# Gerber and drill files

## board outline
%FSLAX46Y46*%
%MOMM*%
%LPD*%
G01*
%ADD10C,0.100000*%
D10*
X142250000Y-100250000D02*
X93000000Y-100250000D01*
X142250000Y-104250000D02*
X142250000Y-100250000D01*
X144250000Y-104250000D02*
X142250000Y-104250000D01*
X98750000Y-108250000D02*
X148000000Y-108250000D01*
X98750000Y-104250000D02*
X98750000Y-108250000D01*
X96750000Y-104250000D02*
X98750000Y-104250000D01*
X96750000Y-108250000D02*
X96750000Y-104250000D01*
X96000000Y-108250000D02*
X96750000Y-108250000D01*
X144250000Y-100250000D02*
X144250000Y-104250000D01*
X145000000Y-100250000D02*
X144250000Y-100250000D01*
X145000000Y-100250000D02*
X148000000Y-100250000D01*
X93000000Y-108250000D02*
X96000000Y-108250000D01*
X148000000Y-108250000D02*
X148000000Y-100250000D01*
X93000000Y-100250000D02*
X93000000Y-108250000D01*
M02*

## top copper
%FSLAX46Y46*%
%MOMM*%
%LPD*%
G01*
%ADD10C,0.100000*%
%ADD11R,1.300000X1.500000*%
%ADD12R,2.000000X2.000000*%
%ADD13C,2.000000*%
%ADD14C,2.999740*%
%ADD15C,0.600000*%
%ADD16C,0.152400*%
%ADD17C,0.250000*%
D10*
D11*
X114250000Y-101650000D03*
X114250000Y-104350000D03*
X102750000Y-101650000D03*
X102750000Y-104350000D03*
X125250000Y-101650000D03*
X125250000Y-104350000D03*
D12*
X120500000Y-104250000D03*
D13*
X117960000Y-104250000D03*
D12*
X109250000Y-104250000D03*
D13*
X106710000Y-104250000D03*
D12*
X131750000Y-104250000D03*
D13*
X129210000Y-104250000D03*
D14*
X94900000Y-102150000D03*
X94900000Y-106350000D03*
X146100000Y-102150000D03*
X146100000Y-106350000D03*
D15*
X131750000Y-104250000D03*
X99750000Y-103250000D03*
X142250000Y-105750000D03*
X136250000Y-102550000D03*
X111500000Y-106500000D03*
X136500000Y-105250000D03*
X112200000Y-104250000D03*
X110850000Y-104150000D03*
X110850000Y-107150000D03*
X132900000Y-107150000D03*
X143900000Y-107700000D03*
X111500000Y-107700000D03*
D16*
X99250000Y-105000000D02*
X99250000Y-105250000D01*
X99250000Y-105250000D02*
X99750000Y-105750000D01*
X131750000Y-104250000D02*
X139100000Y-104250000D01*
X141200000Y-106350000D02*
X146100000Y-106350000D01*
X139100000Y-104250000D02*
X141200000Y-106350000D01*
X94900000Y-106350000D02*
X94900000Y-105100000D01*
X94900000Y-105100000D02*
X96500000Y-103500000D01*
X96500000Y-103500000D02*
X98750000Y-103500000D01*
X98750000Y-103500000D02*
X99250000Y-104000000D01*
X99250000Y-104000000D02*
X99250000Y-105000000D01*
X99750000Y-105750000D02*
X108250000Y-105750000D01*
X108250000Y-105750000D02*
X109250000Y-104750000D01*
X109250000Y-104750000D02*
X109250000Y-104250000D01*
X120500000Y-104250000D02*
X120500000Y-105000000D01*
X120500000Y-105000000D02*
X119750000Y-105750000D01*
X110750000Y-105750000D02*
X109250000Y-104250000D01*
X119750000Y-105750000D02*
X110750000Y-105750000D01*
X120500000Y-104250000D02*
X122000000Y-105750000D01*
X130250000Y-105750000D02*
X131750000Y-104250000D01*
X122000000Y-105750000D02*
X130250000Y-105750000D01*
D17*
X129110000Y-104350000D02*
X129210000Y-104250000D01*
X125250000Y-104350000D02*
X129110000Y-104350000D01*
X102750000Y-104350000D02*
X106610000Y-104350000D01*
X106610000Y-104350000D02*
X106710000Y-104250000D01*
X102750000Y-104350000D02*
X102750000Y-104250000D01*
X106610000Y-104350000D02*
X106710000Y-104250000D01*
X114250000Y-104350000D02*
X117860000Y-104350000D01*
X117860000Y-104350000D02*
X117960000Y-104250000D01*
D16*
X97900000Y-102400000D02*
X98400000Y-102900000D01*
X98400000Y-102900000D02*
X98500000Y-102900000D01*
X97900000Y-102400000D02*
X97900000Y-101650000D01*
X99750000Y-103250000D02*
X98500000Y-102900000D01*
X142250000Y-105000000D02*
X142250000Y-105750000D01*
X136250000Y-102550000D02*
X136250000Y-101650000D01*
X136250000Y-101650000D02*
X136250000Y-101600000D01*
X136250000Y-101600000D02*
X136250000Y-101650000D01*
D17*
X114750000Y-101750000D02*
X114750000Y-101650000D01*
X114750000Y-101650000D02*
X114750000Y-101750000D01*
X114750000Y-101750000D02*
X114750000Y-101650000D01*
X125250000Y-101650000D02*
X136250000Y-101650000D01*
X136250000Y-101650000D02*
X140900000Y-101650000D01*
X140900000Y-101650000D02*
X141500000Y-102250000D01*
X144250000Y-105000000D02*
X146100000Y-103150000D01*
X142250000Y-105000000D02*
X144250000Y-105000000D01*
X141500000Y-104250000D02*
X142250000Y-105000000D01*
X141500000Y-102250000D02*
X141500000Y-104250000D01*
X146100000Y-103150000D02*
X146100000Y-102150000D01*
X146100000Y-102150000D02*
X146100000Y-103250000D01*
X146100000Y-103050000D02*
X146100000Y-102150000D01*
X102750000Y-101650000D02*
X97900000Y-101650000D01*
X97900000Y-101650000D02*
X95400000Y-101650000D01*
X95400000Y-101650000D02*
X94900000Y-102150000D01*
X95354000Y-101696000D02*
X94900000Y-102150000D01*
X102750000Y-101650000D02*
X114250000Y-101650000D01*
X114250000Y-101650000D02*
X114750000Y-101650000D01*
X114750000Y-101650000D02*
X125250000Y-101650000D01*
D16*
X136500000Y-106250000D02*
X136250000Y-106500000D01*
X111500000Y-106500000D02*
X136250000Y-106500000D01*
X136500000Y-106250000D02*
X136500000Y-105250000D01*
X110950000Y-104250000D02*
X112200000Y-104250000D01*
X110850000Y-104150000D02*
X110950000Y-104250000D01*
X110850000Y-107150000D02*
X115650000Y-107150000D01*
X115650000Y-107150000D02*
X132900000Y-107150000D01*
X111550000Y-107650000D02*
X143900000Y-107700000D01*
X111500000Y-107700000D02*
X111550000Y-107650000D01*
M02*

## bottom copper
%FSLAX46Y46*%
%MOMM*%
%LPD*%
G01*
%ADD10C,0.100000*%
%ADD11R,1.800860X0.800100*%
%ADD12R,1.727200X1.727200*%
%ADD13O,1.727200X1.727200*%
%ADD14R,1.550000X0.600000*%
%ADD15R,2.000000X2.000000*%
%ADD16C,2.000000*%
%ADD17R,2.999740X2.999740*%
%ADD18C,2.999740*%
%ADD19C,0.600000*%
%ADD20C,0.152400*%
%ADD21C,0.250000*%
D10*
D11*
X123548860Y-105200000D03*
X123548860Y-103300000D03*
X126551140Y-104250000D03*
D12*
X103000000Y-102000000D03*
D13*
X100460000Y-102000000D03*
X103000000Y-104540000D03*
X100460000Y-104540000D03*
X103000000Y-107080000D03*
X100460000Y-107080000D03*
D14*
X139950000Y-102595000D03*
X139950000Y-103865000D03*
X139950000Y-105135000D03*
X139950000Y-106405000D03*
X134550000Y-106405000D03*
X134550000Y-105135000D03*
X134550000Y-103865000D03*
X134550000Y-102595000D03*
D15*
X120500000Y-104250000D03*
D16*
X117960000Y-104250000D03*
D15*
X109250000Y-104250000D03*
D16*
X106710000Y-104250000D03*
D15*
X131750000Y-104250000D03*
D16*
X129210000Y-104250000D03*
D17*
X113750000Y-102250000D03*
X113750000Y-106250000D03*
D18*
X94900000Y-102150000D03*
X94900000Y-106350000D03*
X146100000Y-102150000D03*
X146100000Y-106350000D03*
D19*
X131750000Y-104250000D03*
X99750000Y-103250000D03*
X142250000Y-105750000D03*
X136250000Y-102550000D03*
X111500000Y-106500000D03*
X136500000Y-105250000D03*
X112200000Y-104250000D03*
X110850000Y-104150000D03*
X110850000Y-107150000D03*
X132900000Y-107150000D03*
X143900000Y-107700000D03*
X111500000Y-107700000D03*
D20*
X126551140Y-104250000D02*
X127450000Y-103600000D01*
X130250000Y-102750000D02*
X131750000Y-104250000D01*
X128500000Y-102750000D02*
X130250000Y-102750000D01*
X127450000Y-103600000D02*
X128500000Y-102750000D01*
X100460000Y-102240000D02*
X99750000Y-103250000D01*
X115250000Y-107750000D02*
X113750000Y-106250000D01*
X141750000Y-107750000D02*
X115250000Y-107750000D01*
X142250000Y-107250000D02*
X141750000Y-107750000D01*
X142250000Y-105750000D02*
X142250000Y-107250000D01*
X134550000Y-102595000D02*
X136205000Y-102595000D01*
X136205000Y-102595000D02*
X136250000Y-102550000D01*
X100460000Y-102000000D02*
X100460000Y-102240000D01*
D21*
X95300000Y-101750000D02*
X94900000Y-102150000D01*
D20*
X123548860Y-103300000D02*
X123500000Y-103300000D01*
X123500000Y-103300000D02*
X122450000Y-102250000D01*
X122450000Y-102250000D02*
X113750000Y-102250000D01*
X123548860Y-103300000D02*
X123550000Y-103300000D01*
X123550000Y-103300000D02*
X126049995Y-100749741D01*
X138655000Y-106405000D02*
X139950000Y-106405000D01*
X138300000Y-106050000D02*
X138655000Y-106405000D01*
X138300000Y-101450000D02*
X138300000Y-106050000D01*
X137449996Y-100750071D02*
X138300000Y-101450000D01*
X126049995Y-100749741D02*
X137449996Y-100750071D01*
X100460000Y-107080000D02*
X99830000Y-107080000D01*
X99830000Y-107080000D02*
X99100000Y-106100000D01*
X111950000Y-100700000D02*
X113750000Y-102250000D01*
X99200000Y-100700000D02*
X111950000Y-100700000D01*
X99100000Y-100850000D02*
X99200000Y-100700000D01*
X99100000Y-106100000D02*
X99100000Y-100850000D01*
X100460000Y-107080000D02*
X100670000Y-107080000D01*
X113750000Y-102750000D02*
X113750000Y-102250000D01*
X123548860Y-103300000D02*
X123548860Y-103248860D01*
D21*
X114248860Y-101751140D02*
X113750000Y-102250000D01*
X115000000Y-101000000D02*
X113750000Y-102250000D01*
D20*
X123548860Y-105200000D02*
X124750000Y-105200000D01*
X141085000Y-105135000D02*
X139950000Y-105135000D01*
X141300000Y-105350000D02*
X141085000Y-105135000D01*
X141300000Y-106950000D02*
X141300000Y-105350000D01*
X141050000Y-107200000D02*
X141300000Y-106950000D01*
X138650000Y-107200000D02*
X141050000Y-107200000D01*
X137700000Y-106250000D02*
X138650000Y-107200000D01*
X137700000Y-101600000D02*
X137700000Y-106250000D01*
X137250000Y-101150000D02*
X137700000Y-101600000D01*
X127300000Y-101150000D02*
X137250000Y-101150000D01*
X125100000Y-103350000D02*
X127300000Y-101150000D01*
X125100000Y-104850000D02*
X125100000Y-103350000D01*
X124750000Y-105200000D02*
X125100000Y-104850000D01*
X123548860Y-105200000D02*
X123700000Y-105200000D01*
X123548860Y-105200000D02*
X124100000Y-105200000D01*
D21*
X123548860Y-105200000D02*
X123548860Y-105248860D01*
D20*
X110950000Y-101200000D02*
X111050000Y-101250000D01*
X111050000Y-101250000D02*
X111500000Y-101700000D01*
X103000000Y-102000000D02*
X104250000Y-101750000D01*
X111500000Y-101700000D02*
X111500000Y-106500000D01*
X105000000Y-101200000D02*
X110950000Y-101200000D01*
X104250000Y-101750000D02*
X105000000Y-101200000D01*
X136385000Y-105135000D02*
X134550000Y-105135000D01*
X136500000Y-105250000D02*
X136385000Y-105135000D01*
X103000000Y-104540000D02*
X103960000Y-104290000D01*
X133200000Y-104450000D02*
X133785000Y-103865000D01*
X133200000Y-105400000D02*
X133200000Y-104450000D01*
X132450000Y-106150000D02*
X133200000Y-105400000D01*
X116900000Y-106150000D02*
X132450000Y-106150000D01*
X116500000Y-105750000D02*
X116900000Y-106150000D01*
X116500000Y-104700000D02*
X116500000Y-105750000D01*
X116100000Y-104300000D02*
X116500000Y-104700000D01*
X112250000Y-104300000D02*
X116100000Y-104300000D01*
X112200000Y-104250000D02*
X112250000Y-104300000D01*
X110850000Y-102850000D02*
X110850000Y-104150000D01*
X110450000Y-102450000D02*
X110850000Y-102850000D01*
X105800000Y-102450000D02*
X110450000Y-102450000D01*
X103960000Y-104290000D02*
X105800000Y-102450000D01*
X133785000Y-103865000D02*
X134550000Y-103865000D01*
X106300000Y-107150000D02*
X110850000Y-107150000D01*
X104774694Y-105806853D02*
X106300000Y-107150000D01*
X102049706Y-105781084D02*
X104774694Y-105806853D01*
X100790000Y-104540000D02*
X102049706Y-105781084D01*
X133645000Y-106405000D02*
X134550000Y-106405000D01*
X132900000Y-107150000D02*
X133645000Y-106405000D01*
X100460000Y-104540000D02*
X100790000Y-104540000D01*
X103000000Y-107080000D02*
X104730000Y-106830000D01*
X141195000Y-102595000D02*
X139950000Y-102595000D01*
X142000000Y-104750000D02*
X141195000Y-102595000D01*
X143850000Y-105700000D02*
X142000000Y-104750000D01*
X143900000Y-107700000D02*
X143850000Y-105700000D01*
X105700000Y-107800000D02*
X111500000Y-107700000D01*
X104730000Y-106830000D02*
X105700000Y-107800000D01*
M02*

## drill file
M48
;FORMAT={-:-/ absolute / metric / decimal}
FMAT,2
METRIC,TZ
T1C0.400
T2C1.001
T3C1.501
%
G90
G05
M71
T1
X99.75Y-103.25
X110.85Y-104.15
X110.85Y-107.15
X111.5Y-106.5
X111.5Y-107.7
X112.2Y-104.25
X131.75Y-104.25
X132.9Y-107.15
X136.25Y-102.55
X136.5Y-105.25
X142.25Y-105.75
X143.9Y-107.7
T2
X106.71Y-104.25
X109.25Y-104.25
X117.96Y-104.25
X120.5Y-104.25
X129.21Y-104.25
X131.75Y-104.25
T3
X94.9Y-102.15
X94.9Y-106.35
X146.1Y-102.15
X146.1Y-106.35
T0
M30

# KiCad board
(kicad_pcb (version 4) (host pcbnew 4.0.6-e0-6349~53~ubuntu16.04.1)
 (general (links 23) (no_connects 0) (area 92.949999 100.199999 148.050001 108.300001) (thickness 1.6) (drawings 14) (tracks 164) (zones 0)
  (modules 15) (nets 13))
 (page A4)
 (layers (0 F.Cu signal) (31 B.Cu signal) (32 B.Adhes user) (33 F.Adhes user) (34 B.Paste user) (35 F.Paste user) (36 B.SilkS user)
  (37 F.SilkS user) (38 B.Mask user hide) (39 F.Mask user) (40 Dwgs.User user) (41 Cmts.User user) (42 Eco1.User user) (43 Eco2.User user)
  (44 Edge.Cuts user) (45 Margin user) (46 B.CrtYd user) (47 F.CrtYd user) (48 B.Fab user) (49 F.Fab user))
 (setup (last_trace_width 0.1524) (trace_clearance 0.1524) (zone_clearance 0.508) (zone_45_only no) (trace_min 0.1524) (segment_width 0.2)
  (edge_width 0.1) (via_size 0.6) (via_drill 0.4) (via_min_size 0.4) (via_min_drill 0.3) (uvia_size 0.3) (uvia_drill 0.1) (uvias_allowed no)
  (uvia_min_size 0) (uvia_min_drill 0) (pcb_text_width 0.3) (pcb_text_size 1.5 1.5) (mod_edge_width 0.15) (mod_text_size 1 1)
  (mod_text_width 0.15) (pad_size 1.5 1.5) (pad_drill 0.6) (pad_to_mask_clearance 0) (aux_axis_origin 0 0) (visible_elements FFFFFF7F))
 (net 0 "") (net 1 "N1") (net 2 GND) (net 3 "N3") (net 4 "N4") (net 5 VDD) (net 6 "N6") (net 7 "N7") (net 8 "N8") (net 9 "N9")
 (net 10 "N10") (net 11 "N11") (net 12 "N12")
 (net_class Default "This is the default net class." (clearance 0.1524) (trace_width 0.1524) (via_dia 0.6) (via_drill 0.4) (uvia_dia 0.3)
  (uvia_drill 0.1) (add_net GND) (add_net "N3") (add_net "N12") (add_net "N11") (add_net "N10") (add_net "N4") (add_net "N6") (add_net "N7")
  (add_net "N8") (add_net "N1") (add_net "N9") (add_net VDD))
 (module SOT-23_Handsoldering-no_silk (layer B.Cu) (at 125.05 104.25 90)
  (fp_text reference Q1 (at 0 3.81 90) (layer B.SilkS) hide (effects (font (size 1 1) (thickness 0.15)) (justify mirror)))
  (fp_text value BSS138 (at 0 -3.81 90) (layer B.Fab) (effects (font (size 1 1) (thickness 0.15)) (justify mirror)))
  (pad 1 smd rect (at -0.95 -1.50114 90) (size 0.8001 1.80086) (layers B.Cu B.Paste B.Mask) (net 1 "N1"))
  (pad 2 smd rect (at 0.95 -1.50114 90) (size 0.8001 1.80086) (layers B.Cu B.Paste B.Mask) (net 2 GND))
  (pad 3 smd rect (at 0 1.50114 90) (size 0.8001 1.80086) (layers B.Cu B.Paste B.Mask) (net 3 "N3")))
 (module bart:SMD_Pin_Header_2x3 (layer B.Cu) (at 103 102 180)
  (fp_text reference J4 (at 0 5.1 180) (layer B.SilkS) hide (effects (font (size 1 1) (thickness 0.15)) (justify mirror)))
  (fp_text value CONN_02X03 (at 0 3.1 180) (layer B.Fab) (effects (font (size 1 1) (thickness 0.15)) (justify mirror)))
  (pad 1 connect rect (at 0 0 180) (size 1.7272 1.7272) (layers B.Cu B.Mask) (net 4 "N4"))
  (pad 2 connect oval (at 2.54 0 180) (size 1.7272 1.7272) (layers B.Cu B.Mask) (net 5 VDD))
  (pad 3 connect oval (at 0 -2.54 180) (size 1.7272 1.7272) (layers B.Cu B.Mask) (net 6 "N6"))
  (pad 4 connect oval (at 2.54 -2.54 180) (size 1.7272 1.7272) (layers B.Cu B.Mask) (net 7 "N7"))
  (pad 5 connect oval (at 0 -5.08 180) (size 1.7272 1.7272) (layers B.Cu B.Mask) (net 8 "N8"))
  (pad 6 connect oval (at 2.54 -5.08 180) (size 1.7272 1.7272) (layers B.Cu B.Mask) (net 2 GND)))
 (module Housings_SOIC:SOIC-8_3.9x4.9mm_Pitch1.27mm (layer B.Cu) (at 137.25 104.5 180)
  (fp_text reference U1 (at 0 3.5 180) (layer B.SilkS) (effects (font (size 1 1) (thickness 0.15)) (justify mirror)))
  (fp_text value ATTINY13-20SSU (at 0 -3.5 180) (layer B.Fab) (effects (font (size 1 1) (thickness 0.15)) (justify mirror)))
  (pad 1 smd rect (at -2.7 1.905 180) (size 1.55 0.6) (layers B.Cu B.Paste B.Mask) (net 8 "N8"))
  (pad 2 smd rect (at -2.7 0.635 180) (size 1.55 0.6) (layers B.Cu B.Paste B.Mask) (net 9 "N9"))
  (pad 3 smd rect (at -2.7 -0.635 180) (size 1.55 0.6) (layers B.Cu B.Paste B.Mask) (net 1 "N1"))
  (pad 4 smd rect (at -2.7 -1.905 180) (size 1.55 0.6) (layers B.Cu B.Paste B.Mask) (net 2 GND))
  (pad 5 smd rect (at 2.7 -1.905 180) (size 1.55 0.6) (layers B.Cu B.Paste B.Mask) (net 7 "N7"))
  (pad 6 smd rect (at 2.7 -0.635 180) (size 1.55 0.6) (layers B.Cu B.Paste B.Mask) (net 4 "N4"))
  (pad 7 smd rect (at 2.7 0.635 180) (size 1.55 0.6) (layers B.Cu B.Paste B.Mask) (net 6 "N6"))
  (pad 8 smd rect (at 2.7 1.905 180) (size 1.55 0.6) (layers B.Cu B.Paste B.Mask) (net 5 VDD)))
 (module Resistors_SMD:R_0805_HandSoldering (layer F.Cu) (at 114.25 103 270)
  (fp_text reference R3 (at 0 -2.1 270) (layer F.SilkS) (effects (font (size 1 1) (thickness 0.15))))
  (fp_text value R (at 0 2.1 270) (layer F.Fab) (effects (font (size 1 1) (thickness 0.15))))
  (pad 1 smd rect (at -1.35 0 270) (size 1.5 1.3) (layers F.Cu F.Paste F.Mask) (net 5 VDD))
  (pad 2 smd rect (at 1.35 0 270) (size 1.5 1.3) (layers F.Cu F.Paste F.Mask) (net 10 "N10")))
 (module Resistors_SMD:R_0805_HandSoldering (layer F.Cu) (at 102.75 103 270)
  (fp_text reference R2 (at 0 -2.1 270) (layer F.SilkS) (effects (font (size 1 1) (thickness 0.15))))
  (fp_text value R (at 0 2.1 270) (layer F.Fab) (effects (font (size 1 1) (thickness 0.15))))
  (pad 1 smd rect (at -1.35 0 270) (size 1.5 1.3) (layers F.Cu F.Paste F.Mask) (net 5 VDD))
  (pad 2 smd rect (at 1.35 0 270) (size 1.5 1.3) (layers F.Cu F.Paste F.Mask) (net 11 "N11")))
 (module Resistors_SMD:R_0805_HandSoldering (layer F.Cu) (at 125.25 103 270)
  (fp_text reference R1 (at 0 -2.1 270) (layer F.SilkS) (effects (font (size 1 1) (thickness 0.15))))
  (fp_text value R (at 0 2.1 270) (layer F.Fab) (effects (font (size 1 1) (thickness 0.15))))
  (pad 1 smd rect (at -1.35 0 270) (size 1.5 1.3) (layers F.Cu F.Paste F.Mask) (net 5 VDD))
  (pad 2 smd rect (at 1.35 0 270) (size 1.5 1.3) (layers F.Cu F.Paste F.Mask) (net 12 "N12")))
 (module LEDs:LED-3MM (layer F.Cu) (at 120.5 104.25 180)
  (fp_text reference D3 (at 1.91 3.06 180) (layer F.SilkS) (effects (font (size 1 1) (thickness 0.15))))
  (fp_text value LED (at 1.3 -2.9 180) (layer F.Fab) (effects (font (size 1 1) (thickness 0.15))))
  (pad 1 thru_hole rect (at 0 0 270) (size 2 2) (drill 1.00076) (layers *.Cu *.Mask F.SilkS) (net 3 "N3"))
  (pad 2 thru_hole circle (at 2.54 0 180) (size 2 2) (drill 1.00076) (layers *.Cu *.Mask F.SilkS) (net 10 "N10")))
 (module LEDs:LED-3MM (layer F.Cu) (at 109.25 104.25 180)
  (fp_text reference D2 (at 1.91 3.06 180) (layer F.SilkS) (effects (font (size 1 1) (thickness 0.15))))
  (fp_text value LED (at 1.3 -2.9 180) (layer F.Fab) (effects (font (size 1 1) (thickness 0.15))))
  (pad 1 thru_hole rect (at 0 0 270) (size 2 2) (drill 1.00076) (layers *.Cu *.Mask F.SilkS) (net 3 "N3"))
  (pad 2 thru_hole circle (at 2.54 0 180) (size 2 2) (drill 1.00076) (layers *.Cu *.Mask F.SilkS) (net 11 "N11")))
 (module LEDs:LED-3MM (layer F.Cu) (at 131.75 104.25 180)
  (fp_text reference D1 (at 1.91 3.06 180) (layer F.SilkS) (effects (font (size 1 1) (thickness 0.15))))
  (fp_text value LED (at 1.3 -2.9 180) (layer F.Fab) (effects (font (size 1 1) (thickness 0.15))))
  (pad 1 thru_hole rect (at 0 0 270) (size 2 2) (drill 1.00076) (layers *.Cu *.Mask F.SilkS) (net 3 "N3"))
  (pad 2 thru_hole circle (at 2.54 0 180) (size 2 2) (drill 1.00076) (layers *.Cu *.Mask F.SilkS) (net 12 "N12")))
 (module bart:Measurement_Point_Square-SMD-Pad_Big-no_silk (layer B.Cu) (at 113.75 102.25)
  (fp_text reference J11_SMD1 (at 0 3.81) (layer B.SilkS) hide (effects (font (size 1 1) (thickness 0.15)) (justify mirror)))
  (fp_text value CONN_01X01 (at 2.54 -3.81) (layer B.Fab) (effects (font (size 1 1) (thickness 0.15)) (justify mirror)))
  (pad 1 smd rect (at 0 0) (size 2.99974 2.99974) (layers B.Cu B.Paste B.Mask) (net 2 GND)))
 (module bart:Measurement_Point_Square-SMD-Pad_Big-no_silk (layer B.Cu) (at 113.75 106.25)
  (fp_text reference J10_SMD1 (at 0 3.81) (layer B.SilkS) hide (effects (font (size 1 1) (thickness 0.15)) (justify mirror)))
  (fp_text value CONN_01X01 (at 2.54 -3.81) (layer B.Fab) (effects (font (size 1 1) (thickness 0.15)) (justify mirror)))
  (pad 1 smd rect (at 0 0) (size 2.99974 2.99974) (layers B.Cu B.Paste B.Mask) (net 5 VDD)))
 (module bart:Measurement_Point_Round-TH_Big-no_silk (layer F.Cu) (at 94.9 102.15)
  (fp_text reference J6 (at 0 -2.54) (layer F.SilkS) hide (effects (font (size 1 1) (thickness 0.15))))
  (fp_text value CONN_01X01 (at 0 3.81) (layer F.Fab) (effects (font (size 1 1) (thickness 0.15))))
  (pad 1 thru_hole circle (at 0 0) (size 2.99974 2.99974) (drill 1.50114) (layers *.Cu *.Mask F.SilkS) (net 5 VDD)))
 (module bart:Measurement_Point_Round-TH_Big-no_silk (layer F.Cu) (at 94.9 106.35)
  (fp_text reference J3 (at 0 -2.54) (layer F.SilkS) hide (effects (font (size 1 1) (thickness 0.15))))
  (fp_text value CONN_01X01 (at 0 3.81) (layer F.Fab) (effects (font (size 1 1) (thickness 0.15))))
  (pad 1 thru_hole circle (at 0 0) (size 2.99974 2.99974) (drill 1.50114) (layers *.Cu *.Mask F.SilkS) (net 3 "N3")))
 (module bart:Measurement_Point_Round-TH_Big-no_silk (layer F.Cu) (at 146.1 102.15)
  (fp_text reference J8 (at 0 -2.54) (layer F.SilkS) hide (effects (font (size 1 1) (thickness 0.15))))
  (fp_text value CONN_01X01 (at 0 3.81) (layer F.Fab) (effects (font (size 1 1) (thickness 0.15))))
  (pad 1 thru_hole circle (at 0 0) (size 2.99974 2.99974) (drill 1.50114) (layers *.Cu *.Mask F.SilkS) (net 5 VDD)))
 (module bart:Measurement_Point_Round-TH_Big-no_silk (layer F.Cu) (at 146.1 106.35)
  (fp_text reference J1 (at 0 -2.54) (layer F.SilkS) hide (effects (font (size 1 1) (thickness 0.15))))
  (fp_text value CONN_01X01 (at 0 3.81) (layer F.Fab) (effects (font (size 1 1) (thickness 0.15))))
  (pad 1 thru_hole circle (at 0 0) (size 2.99974 2.99974) (drill 1.50114) (layers *.Cu *.Mask F.SilkS) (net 3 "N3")))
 (gr_line (start 142.25 100.25) (end 93 100.25) (angle 90) (layer Edge.Cuts) (width 0.1))
 (gr_line (start 142.25 104.25) (end 142.25 100.25) (angle 90) (layer Edge.Cuts) (width 0.1))
 (gr_line (start 144.25 104.25) (end 142.25 104.25) (angle 90) (layer Edge.Cuts) (width 0.1))
 (gr_line (start 98.75 108.25) (end 148 108.25) (angle 90) (layer Edge.Cuts) (width 0.1))
 (gr_line (start 98.75 104.25) (end 98.75 108.25) (angle 90) (layer Edge.Cuts) (width 0.1))
 (gr_line (start 96.75 104.25) (end 98.75 104.25) (angle 90) (layer Edge.Cuts) (width 0.1))
 (gr_line (start 96.75 108.25) (end 96.75 104.25) (angle 90) (layer Edge.Cuts) (width 0.1))
 (gr_line (start 96 108.25) (end 96.75 108.25) (angle 90) (layer Edge.Cuts) (width 0.1))
 (gr_line (start 144.25 100.25) (end 144.25 104.25) (angle 90) (layer Edge.Cuts) (width 0.1))
 (gr_line (start 145 100.25) (end 144.25 100.25) (angle 90) (layer Edge.Cuts) (width 0.1))
 (gr_line (start 145 100.25) (end 148 100.25) (angle 90) (layer Edge.Cuts) (width 0.1))
 (gr_line (start 93 108.25) (end 96 108.25) (angle 90) (layer Edge.Cuts) (width 0.1))
 (gr_line (start 148 108.25) (end 148 100.25) (angle 90) (layer Edge.Cuts) (width 0.1))
 (gr_line (start 93 100.25) (end 93 108.25) (angle 90) (layer Edge.Cuts) (width 0.1))
 (segment (start 99.25 105) (end 99.25 105.25) (width 0.1524) (layer F.Cu) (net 3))
 (segment (start 99.25 105.25) (end 99.75 105.75) (width 0.1524) (layer F.Cu) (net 3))
 (segment (start 131.75 104.25) (end 139.1 104.25) (width 0.1524) (layer F.Cu) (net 3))
 (segment (start 141.2 106.35) (end 146.1 106.35) (width 0.1524) (layer F.Cu) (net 3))
 (segment (start 139.1 104.25) (end 141.2 106.35) (width 0.1524) (layer F.Cu) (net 3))
 (segment (start 126.55114 104.25) (end 127.45 103.6) (width 0.1524) (layer B.Cu) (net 3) (status 10))
 (segment (start 130.25 102.75) (end 131.75 104.25) (width 0.1524) (layer B.Cu) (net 3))
 (segment (start 128.5 102.75) (end 130.25 102.75) (width 0.1524) (layer B.Cu) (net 3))
 (segment (start 127.45 103.6) (end 128.5 102.75) (width 0.1524) (layer B.Cu) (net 3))
 (segment (start 94.9 106.35) (end 94.9 105.1) (width 0.1524) (layer F.Cu) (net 3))
 (segment (start 94.9 105.1) (end 96.5 103.5) (width 0.1524) (layer F.Cu) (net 3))
 (segment (start 96.5 103.5) (end 98.75 103.5) (width 0.1524) (layer F.Cu) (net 3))
 (segment (start 98.75 103.5) (end 99.25 104) (width 0.1524) (layer F.Cu) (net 3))
 (segment (start 99.25 104) (end 99.25 105) (width 0.1524) (layer F.Cu) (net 3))
 (segment (start 99.75 105.75) (end 108.25 105.75) (width 0.1524) (layer F.Cu) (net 3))
 (segment (start 108.25 105.75) (end 109.25 104.75) (width 0.1524) (layer F.Cu) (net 3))
 (segment (start 109.25 104.75) (end 109.25 104.25) (width 0.1524) (layer F.Cu) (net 3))
 (segment (start 120.5 104.25) (end 120.5 105) (width 0.1524) (layer F.Cu) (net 3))
 (segment (start 120.5 105) (end 119.75 105.75) (width 0.1524) (layer F.Cu) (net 3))
 (segment (start 110.75 105.75) (end 109.25 104.25) (width 0.1524) (layer F.Cu) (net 3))
 (segment (start 119.75 105.75) (end 110.75 105.75) (width 0.1524) (layer F.Cu) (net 3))
 (segment (start 120.5 104.25) (end 122 105.75) (width 0.1524) (layer F.Cu) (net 3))
 (segment (start 130.25 105.75) (end 131.75 104.25) (width 0.1524) (layer F.Cu) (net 3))
 (segment (start 122 105.75) (end 130.25 105.75) (width 0.1524) (layer F.Cu) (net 3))
 (via (at 131.75 104.25) (size 0.6) (drill 0.4) (layers F.Cu B.Cu) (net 3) (status 30))
 (segment (start 129.11 104.35) (end 129.21 104.25) (width 0.25) (layer F.Cu) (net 12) (status 30))
 (segment (start 125.25 104.35) (end 129.11 104.35) (width 0.25) (layer F.Cu) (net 12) (status 20))
 (segment (start 102.75 104.35) (end 106.61 104.35) (width 0.25) (layer F.Cu) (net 11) (status 20))
 (segment (start 106.61 104.35) (end 106.71 104.25) (width 0.25) (layer F.Cu) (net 11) (status 30))
 (segment (start 102.75 104.35) (end 102.75 104.25) (width 0.25) (layer F.Cu) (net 11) (status 30))
 (segment (start 106.61 104.35) (end 106.71 104.25) (width 0.25) (layer F.Cu) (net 11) (status 30))
 (segment (start 114.25 104.35) (end 117.86 104.35) (width 0.25) (layer F.Cu) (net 10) (status 10))
 (segment (start 117.86 104.35) (end 117.96 104.25) (width 0.25) (layer F.Cu) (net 10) (status 30))
 (segment (start 97.9 102.4) (end 98.4 102.9) (width 0.1524) (layer F.Cu) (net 5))
 (segment (start 98.4 102.9) (end 98.5 102.9) (width 0.1524) (layer F.Cu) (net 5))
 (segment (start 97.9 102.4) (end 97.9 101.65) (width 0.1524) (layer F.Cu) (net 5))
 (segment (start 100.46 102.24) (end 99.75 103.25) (width 0.1524) (layer B.Cu) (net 5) (status 10))
 (via (at 99.75 103.25) (size 0.6) (drill 0.4) (layers F.Cu B.Cu) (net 5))
 (segment (start 99.75 103.25) (end 98.5 102.9) (width 0.1524) (layer F.Cu) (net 5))
 (segment (start 142.25 105) (end 142.25 105.75) (width 0.1524) (layer F.Cu) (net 5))
 (segment (start 115.25 107.75) (end 113.75 106.25) (width 0.1524) (layer B.Cu) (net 5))
 (segment (start 141.75 107.75) (end 115.25 107.75) (width 0.1524) (layer B.Cu) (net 5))
 (segment (start 142.25 107.25) (end 141.75 107.75) (width 0.1524) (layer B.Cu) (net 5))
 (segment (start 142.25 105.75) (end 142.25 107.25) (width 0.1524) (layer B.Cu) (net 5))
 (via (at 142.25 105.75) (size 0.6) (drill 0.4) (layers F.Cu B.Cu) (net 5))
 (segment (start 134.55 102.595) (end 136.205 102.595) (width 0.1524) (layer B.Cu) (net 5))
 (segment (start 136.25 102.55) (end 136.25 101.65) (width 0.1524) (layer F.Cu) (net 5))
 (via (at 136.25 102.55) (size 0.6) (drill 0.4) (layers F.Cu B.Cu) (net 5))
 (segment (start 136.205 102.595) (end 136.25 102.55) (width 0.1524) (layer B.Cu) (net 5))
 (segment (start 136.25 101.65) (end 136.25 101.6) (width 0.1524) (layer F.Cu) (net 5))
 (segment (start 136.25 101.6) (end 136.25 101.65) (width 0.1524) (layer F.Cu) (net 5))
 (segment (start 100.46 102) (end 100.46 102.24) (width 0.1524) (layer B.Cu) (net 5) (status 30))
 (segment (start 95.3 101.75) (end 94.9 102.15) (width 0.25) (layer B.Cu) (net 5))
 (segment (start 114.75 101.75) (end 114.75 101.65) (width 0.25) (layer F.Cu) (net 5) (status 30))
 (segment (start 114.75 101.65) (end 114.75 101.75) (width 0.25) (layer F.Cu) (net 5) (status 30))
 (segment (start 114.75 101.75) (end 114.75 101.65) (width 0.25) (layer F.Cu) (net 5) (status 30))
 (segment (start 125.25 101.65) (end 136.25 101.65) (width 0.25) (layer F.Cu) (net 5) (status 10))
 (segment (start 136.25 101.65) (end 140.9 101.65) (width 0.25) (layer F.Cu) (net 5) (status 10))
 (segment (start 140.9 101.65) (end 141.5 102.25) (width 0.25) (layer F.Cu) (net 5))
 (segment (start 144.25 105) (end 146.1 103.15) (width 0.25) (layer F.Cu) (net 5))
 (segment (start 142.25 105) (end 144.25 105) (width 0.25) (layer F.Cu) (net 5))
 (segment (start 141.5 104.25) (end 142.25 105) (width 0.25) (layer F.Cu) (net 5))
 (segment (start 141.5 102.25) (end 141.5 104.25) (width 0.25) (layer F.Cu) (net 5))
 (segment (start 146.1 103.15) (end 146.1 102.15) (width 0.25) (layer F.Cu) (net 5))
 (segment (start 146.1 102.15) (end 146.1 103.25) (width 0.25) (layer F.Cu) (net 5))
 (segment (start 146.1 103.05) (end 146.1 102.15) (width 0.25) (layer F.Cu) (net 5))
 (segment (start 102.75 101.65) (end 97.9 101.65) (width 0.25) (layer F.Cu) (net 5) (status 10))
 (segment (start 97.9 101.65) (end 95.4 101.65) (width 0.25) (layer F.Cu) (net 5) (status 10))
 (segment (start 95.4 101.65) (end 94.9 102.15) (width 0.25) (layer F.Cu) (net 5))
 (segment (start 95.354 101.696) (end 94.9 102.15) (width 0.25) (layer F.Cu) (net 5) (status 30))
 (segment (start 102.75 101.65) (end 114.25 101.65) (width 0.25) (layer F.Cu) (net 5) (status 20))
 (segment (start 114.25 101.65) (end 114.75 101.65) (width 0.25) (layer F.Cu) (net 5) (status 30))
 (segment (start 114.75 101.65) (end 125.25 101.65) (width 0.25) (layer F.Cu) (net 5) (status 10))
 (segment (start 123.54886 103.3) (end 123.5 103.3) (width 0.1524) (layer B.Cu) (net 2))
 (segment (start 123.5 103.3) (end 122.45 102.25) (width 0.1524) (layer B.Cu) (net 2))
 (segment (start 122.45 102.25) (end 113.75 102.25) (width 0.1524) (layer B.Cu) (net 2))
 (segment (start 123.54886 103.3) (end 123.55 103.3) (width 0.1524) (layer B.Cu) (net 2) (status 30))
 (segment (start 123.55 103.3) (end 126.049995 100.749741) (width 0.1524) (layer B.Cu) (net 2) (status 10))
 (segment (start 138.655 106.405) (end 139.95 106.405) (width 0.1524) (layer B.Cu) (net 2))
 (segment (start 138.3 106.05) (end 138.655 106.405) (width 0.1524) (layer B.Cu) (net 2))
 (segment (start 138.3 101.45) (end 138.3 106.05) (width 0.1524) (layer B.Cu) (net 2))
 (segment (start 137.449996 100.750071) (end 138.3 101.45) (width 0.1524) (layer B.Cu) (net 2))
 (segment (start 126.049995 100.749741) (end 137.449996 100.750071) (width 0.1524) (layer B.Cu) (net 2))
 (segment (start 100.46 107.08) (end 99.83 107.08) (width 0.1524) (layer B.Cu) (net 2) (status 30))
 (segment (start 99.83 107.08) (end 99.1 106.1) (width 0.1524) (layer B.Cu) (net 2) (status 10))
 (segment (start 111.95 100.7) (end 113.75 102.25) (width 0.1524) (layer B.Cu) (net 2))
 (segment (start 99.2 100.7) (end 111.95 100.7) (width 0.1524) (layer B.Cu) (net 2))
 (segment (start 99.1 100.85) (end 99.2 100.7) (width 0.1524) (layer B.Cu) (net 2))
 (segment (start 99.1 106.1) (end 99.1 100.85) (width 0.1524) (layer B.Cu) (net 2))
 (segment (start 100.46 107.08) (end 100.67 107.08) (width 0.1524) (layer B.Cu) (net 2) (status 30))
 (segment (start 113.75 102.75) (end 113.75 102.25) (width 0.1524) (layer B.Cu) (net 2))
 (segment (start 123.54886 103.3) (end 123.54886 103.24886) (width 0.1524) (layer B.Cu) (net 2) (status 30))
 (segment (start 114.24886 101.75114) (end 113.75 102.25) (width 0.25) (layer B.Cu) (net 2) (status 30))
 (segment (start 115 101) (end 113.75 102.25) (width 0.25) (layer B.Cu) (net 2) (status 30))
 (segment (start 123.54886 105.2) (end 124.75 105.2) (width 0.1524) (layer B.Cu) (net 1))
 (segment (start 141.085 105.135) (end 139.95 105.135) (width 0.1524) (layer B.Cu) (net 1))
 (segment (start 141.3 105.35) (end 141.085 105.135) (width 0.1524) (layer B.Cu) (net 1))
 (segment (start 141.3 106.95) (end 141.3 105.35) (width 0.1524) (layer B.Cu) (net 1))
 (segment (start 141.05 107.2) (end 141.3 106.95) (width 0.1524) (layer B.Cu) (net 1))
 (segment (start 138.65 107.2) (end 141.05 107.2) (width 0.1524) (layer B.Cu) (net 1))
 (segment (start 137.7 106.25) (end 138.65 107.2) (width 0.1524) (layer B.Cu) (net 1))
 (segment (start 137.7 101.6) (end 137.7 106.25) (width 0.1524) (layer B.Cu) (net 1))
 (segment (start 137.25 101.15) (end 137.7 101.6) (width 0.1524) (layer B.Cu) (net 1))
 (segment (start 127.3 101.15) (end 137.25 101.15) (width 0.1524) (layer B.Cu) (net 1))
 (segment (start 125.1 103.35) (end 127.3 101.15) (width 0.1524) (layer B.Cu) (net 1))
 (segment (start 125.1 104.85) (end 125.1 103.35) (width 0.1524) (layer B.Cu) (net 1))
 (segment (start 124.75 105.2) (end 125.1 104.85) (width 0.1524) (layer B.Cu) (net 1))
 (segment (start 123.54886 105.2) (end 123.7 105.2) (width 0.1524) (layer B.Cu) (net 1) (status 30))
 (segment (start 123.54886 105.2) (end 124.1 105.2) (width 0.1524) (layer B.Cu) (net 1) (status 30))
 (segment (start 123.54886 105.2) (end 123.54886 105.24886) (width 0.25) (layer B.Cu) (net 1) (status 30))
 (segment (start 136.5 106.25) (end 136.25 106.5) (width 0.1524) (layer F.Cu) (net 4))
 (segment (start 110.95 101.2) (end 111.05 101.25) (width 0.1524) (layer B.Cu) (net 4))
 (segment (start 111.05 101.25) (end 111.5 101.7) (width 0.1524) (layer B.Cu) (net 4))
 (segment (start 103 102) (end 104.25 101.75) (width 0.1524) (layer B.Cu) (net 4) (status 10))
 (segment (start 111.5 106.5) (end 136.25 106.5) (width 0.1524) (layer F.Cu) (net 4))
 (via (at 111.5 106.5) (size 0.6) (drill 0.4) (layers F.Cu B.Cu) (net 4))
 (segment (start 111.5 101.7) (end 111.5 106.5) (width 0.1524) (layer B.Cu) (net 4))
 (segment (start 105 101.2) (end 110.95 101.2) (width 0.1524) (layer B.Cu) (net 4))
 (segment (start 104.25 101.75) (end 105 101.2) (width 0.1524) (layer B.Cu) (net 4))
 (segment (start 136.385 105.135) (end 134.55 105.135) (width 0.1524) (layer B.Cu) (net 4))
 (segment (start 136.5 105.25) (end 136.385 105.135) (width 0.1524) (layer B.Cu) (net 4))
 (via (at 136.5 105.25) (size 0.6) (drill 0.4) (layers F.Cu B.Cu) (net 4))
 (segment (start 136.5 106.25) (end 136.5 105.25) (width 0.1524) (layer F.Cu) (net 4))
 (segment (start 103 104.54) (end 103.96 104.29) (width 0.1524) (layer B.Cu) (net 6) (status 10))
 (segment (start 133.2 104.45) (end 133.785 103.865) (width 0.1524) (layer B.Cu) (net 6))
 (segment (start 133.2 105.4) (end 133.2 104.45) (width 0.1524) (layer B.Cu) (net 6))
 (segment (start 132.45 106.15) (end 133.2 105.4) (width 0.1524) (layer B.Cu) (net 6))
 (segment (start 116.9 106.15) (end 132.45 106.15) (width 0.1524) (layer B.Cu) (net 6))
 (segment (start 116.5 105.75) (end 116.9 106.15) (width 0.1524) (layer B.Cu) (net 6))
 (segment (start 116.5 104.7) (end 116.5 105.75) (width 0.1524) (layer B.Cu) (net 6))
 (segment (start 116.1 104.3) (end 116.5 104.7) (width 0.1524) (layer B.Cu) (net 6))
 (segment (start 112.25 104.3) (end 116.1 104.3) (width 0.1524) (layer B.Cu) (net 6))
 (segment (start 112.2 104.25) (end 112.25 104.3) (width 0.1524) (layer B.Cu) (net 6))
 (via (at 112.2 104.25) (size 0.6) (drill 0.4) (layers F.Cu B.Cu) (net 6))
 (segment (start 110.95 104.25) (end 112.2 104.25) (width 0.1524) (layer F.Cu) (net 6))
 (segment (start 110.85 104.15) (end 110.95 104.25) (width 0.1524) (layer F.Cu) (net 6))
 (via (at 110.85 104.15) (size 0.6) (drill 0.4) (layers F.Cu B.Cu) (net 6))
 (segment (start 110.85 102.85) (end 110.85 104.15) (width 0.1524) (layer B.Cu) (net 6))
 (segment (start 110.45 102.45) (end 110.85 102.85) (width 0.1524) (layer B.Cu) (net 6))
 (segment (start 105.8 102.45) (end 110.45 102.45) (width 0.1524) (layer B.Cu) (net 6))
 (segment (start 103.96 104.29) (end 105.8 102.45) (width 0.1524) (layer B.Cu) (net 6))
 (segment (start 133.785 103.865) (end 134.55 103.865) (width 0.1524) (layer B.Cu) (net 6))
 (segment (start 110.85 107.15) (end 115.65 107.15) (width 0.1524) (layer F.Cu) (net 7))
 (via (at 110.85 107.15) (size 0.6) (drill 0.4) (layers F.Cu B.Cu) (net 7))
 (segment (start 106.3 107.15) (end 110.85 107.15) (width 0.1524) (layer B.Cu) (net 7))
 (segment (start 104.774694 105.806853) (end 106.3 107.15) (width 0.1524) (layer B.Cu) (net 7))
 (segment (start 102.049706 105.781084) (end 104.774694 105.806853) (width 0.1524) (layer B.Cu) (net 7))
 (segment (start 100.79 104.54) (end 102.049706 105.781084) (width 0.1524) (layer B.Cu) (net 7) (status 10))
 (segment (start 133.645 106.405) (end 134.55 106.405) (width 0.1524) (layer B.Cu) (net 7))
 (segment (start 132.9 107.15) (end 133.645 106.405) (width 0.1524) (layer B.Cu) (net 7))
 (via (at 132.9 107.15) (size 0.6) (drill 0.4) (layers F.Cu B.Cu) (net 7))
 (segment (start 115.65 107.15) (end 132.9 107.15) (width 0.1524) (layer F.Cu) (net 7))
 (segment (start 100.46 104.54) (end 100.79 104.54) (width 0.1524) (layer B.Cu) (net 7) (status 30))
 (segment (start 103 107.08) (end 104.73 106.83) (width 0.1524) (layer B.Cu) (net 8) (status 10))
 (segment (start 141.195 102.595) (end 139.95 102.595) (width 0.1524) (layer B.Cu) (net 8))
 (segment (start 142 104.75) (end 141.195 102.595) (width 0.1524) (layer B.Cu) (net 8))
 (segment (start 143.85 105.7) (end 142 104.75) (width 0.1524) (layer B.Cu) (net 8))
 (segment (start 143.9 107.7) (end 143.85 105.7) (width 0.1524) (layer B.Cu) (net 8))
 (via (at 143.9 107.7) (size 0.6) (drill 0.4) (layers F.Cu B.Cu) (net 8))
 (segment (start 111.55 107.65) (end 143.9 107.7) (width 0.1524) (layer F.Cu) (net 8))
 (segment (start 111.5 107.7) (end 111.55 107.65) (width 0.1524) (layer F.Cu) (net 8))
 (via (at 111.5 107.7) (size 0.6) (drill 0.4) (layers F.Cu B.Cu) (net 8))
 (segment (start 105.7 107.8) (end 111.5 107.7) (width 0.1524) (layer B.Cu) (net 8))
 (segment (start 104.73 106.83) (end 105.7 107.8) (width 0.1524) (layer B.Cu) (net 8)))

